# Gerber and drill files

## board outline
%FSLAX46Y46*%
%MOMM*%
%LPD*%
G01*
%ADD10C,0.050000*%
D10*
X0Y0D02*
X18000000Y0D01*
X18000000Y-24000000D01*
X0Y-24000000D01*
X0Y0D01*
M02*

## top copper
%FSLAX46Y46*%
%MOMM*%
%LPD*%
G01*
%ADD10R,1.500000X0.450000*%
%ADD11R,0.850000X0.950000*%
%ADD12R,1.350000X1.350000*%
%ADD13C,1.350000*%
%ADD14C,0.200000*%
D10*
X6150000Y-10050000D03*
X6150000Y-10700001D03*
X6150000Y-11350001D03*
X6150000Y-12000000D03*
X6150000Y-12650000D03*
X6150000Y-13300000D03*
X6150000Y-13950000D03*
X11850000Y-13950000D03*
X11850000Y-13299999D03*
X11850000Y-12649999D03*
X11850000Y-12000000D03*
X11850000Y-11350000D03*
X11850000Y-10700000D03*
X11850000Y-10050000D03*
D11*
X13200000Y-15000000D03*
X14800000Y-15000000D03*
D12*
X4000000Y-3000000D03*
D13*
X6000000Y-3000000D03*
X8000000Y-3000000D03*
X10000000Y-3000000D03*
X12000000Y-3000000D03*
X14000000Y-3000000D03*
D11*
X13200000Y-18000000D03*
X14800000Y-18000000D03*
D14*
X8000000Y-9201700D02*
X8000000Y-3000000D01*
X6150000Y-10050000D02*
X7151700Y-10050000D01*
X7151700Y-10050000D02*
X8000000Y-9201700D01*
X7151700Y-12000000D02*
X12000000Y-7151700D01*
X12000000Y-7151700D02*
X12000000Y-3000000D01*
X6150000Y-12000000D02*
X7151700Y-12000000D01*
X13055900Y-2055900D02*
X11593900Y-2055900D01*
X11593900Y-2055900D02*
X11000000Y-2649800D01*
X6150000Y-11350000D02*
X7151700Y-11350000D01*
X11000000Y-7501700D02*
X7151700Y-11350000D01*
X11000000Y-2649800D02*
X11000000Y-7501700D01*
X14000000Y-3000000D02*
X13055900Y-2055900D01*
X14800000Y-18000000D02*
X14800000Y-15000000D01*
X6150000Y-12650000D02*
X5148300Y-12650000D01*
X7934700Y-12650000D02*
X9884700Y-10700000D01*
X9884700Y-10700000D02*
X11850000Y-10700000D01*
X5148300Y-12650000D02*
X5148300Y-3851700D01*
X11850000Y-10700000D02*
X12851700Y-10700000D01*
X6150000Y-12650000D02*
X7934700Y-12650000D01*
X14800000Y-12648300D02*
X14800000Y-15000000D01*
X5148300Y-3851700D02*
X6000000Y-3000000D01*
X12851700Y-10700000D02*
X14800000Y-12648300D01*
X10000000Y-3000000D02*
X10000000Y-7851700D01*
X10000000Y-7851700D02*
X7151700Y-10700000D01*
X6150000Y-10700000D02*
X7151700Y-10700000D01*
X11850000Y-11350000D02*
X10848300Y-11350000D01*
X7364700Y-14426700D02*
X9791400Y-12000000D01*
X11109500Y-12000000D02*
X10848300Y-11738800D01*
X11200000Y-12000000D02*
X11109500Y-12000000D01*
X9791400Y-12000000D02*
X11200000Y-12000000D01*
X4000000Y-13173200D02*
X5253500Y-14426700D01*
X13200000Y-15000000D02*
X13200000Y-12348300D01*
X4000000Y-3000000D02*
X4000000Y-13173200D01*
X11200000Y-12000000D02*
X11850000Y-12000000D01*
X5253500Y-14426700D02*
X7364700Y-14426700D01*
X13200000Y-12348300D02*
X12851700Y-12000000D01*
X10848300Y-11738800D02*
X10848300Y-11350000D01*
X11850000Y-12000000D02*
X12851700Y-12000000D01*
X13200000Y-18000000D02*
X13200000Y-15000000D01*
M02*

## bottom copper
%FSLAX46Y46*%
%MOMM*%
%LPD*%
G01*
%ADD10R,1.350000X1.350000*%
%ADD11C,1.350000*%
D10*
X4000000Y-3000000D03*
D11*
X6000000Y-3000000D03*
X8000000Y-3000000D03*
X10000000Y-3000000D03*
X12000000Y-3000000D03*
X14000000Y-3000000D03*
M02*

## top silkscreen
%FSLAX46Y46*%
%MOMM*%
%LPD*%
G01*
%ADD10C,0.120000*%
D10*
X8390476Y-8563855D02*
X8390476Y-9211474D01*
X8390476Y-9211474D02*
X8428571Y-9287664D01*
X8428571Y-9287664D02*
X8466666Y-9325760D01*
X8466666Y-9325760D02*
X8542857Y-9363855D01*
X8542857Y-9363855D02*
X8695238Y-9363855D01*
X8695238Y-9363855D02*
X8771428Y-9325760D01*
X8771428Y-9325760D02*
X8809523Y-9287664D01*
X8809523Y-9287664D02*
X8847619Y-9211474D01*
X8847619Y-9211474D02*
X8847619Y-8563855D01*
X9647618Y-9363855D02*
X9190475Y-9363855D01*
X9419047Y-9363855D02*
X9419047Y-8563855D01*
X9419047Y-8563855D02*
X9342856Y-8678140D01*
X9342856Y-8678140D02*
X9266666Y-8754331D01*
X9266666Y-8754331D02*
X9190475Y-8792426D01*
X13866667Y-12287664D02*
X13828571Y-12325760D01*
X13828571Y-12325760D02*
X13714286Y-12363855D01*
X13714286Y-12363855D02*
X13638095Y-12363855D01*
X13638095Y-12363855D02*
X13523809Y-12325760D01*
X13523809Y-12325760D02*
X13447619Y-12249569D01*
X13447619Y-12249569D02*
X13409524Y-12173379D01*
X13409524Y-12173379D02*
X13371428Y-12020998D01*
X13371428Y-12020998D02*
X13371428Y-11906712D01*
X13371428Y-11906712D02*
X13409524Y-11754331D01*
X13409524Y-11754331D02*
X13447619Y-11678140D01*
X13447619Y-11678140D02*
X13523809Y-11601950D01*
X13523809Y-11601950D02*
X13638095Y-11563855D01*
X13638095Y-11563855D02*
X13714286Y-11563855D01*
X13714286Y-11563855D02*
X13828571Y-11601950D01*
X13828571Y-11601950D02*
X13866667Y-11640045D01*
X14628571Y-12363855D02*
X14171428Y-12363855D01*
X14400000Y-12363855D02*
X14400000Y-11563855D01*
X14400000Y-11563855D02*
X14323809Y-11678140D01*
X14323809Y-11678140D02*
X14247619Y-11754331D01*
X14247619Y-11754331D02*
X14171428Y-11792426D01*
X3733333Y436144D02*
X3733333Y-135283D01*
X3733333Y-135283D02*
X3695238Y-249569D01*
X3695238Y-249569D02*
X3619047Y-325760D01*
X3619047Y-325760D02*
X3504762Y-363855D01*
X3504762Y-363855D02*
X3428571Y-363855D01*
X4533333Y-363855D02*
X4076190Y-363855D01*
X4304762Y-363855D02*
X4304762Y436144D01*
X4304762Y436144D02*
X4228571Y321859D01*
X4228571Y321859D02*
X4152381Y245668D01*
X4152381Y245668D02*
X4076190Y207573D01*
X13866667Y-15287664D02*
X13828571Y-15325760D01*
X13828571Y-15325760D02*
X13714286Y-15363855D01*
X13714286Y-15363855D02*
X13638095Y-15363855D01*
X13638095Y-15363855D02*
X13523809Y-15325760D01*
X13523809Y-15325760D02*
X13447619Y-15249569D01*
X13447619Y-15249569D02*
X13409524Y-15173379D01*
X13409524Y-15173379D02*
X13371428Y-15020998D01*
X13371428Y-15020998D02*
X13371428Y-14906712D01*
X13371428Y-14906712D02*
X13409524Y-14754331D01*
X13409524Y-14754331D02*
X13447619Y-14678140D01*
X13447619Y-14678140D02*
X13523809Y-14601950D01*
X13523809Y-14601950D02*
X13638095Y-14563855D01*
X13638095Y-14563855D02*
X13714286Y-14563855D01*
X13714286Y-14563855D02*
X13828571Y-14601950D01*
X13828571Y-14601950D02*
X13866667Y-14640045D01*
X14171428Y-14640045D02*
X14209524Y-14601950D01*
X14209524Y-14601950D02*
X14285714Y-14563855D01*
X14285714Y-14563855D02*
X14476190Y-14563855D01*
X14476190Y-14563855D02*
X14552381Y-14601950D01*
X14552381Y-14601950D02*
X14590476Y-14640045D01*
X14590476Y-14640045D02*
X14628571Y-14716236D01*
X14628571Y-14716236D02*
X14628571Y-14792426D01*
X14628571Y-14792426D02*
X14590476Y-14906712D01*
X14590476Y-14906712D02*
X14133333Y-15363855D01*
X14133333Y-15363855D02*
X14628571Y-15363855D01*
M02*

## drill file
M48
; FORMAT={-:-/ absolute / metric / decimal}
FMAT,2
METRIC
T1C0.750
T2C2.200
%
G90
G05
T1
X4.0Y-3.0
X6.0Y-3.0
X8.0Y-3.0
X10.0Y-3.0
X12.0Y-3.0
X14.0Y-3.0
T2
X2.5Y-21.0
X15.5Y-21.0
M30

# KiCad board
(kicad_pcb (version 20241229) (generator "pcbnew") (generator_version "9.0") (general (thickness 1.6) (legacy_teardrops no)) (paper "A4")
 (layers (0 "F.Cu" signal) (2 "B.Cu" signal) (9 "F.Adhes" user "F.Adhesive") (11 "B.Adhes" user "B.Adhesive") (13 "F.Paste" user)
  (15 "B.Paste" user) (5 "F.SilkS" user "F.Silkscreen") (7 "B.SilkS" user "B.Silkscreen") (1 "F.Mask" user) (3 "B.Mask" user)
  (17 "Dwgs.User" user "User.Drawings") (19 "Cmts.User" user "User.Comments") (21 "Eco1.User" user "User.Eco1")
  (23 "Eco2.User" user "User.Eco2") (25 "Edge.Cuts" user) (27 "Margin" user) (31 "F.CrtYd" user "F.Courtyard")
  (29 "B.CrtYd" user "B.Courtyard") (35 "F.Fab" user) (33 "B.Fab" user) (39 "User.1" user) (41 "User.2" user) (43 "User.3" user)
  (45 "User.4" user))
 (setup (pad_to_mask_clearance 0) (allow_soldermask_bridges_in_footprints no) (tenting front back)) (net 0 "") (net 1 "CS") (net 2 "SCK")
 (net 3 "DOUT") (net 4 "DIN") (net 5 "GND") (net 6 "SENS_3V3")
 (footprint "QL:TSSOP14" (layer "F.Cu") (at 9 12)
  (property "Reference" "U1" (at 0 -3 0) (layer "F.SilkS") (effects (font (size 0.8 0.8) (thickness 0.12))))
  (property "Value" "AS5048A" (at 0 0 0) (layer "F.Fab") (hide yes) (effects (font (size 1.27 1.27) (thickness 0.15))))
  (pad "1" smd rect (at -2.85 -1.95) (size 1.5 0.45) (layers "F.Cu" "F.Mask" "F.Paste") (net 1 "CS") (thermal_bridge_angle 45))
  (pad "2" smd rect (at -2.85 -1.299999) (size 1.5 0.45) (layers "F.Cu" "F.Mask" "F.Paste") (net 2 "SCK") (thermal_bridge_angle 45))
  (pad "3" smd rect (at -2.85 -0.649999) (size 1.5 0.45) (layers "F.Cu" "F.Mask" "F.Paste") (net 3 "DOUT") (thermal_bridge_angle 45))
  (pad "4" smd rect (at -2.85 0) (size 1.5 0.45) (layers "F.Cu" "F.Mask" "F.Paste") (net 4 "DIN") (thermal_bridge_angle 45))
  (pad "5" smd rect (at -2.85 0.65) (size 1.5 0.45) (layers "F.Cu" "F.Mask" "F.Paste") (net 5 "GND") (thermal_bridge_angle 45))
  (pad "6" smd rect (at -2.85 1.3) (size 1.5 0.45) (layers "F.Cu" "F.Mask" "F.Paste") (thermal_bridge_angle 45))
  (pad "7" smd rect (at -2.85 1.95) (size 1.5 0.45) (layers "F.Cu" "F.Mask" "F.Paste") (thermal_bridge_angle 45))
  (pad "8" smd rect (at 2.85 1.95) (size 1.5 0.45) (layers "F.Cu" "F.Mask" "F.Paste") (thermal_bridge_angle 45))
  (pad "9" smd rect (at 2.85 1.299999) (size 1.5 0.45) (layers "F.Cu" "F.Mask" "F.Paste") (thermal_bridge_angle 45))
  (pad "10" smd rect (at 2.85 0.649999) (size 1.5 0.45) (layers "F.Cu" "F.Mask" "F.Paste") (thermal_bridge_angle 45))
  (pad "11" smd rect (at 2.85 0) (size 1.5 0.45) (layers "F.Cu" "F.Mask" "F.Paste") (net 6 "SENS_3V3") (thermal_bridge_angle 45))
  (pad "12" smd rect (at 2.85 -0.65) (size 1.5 0.45) (layers "F.Cu" "F.Mask" "F.Paste") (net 6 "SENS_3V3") (thermal_bridge_angle 45))
  (pad "13" smd rect (at 2.85 -1.3) (size 1.5 0.45) (layers "F.Cu" "F.Mask" "F.Paste") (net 5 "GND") (thermal_bridge_angle 45))
  (pad "14" smd rect (at 2.85 -1.95) (size 1.5 0.45) (layers "F.Cu" "F.Mask" "F.Paste") (thermal_bridge_angle 45)))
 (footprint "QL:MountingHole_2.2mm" (layer "F.Cu") (at 15.5 21)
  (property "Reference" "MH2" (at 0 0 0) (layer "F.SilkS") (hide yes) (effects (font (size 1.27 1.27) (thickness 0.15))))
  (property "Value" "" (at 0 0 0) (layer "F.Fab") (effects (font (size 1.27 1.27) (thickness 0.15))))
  (pad "" np_thru_hole circle (at 0 0) (size 2.2 2.2) (drill 2.2) (layers "*.Cu" "*.Mask")))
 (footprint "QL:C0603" (layer "F.Cu") (at 14 15)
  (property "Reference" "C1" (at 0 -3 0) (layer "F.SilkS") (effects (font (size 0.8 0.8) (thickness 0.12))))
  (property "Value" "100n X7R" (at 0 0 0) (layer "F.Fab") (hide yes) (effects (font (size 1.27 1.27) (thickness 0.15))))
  (pad "1" smd rect (at -0.8 0) (size 0.85 0.95) (layers "F.Cu" "F.Mask" "F.Paste") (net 6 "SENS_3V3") (thermal_bridge_angle 45))
  (pad "2" smd rect (at 0.8 0) (size 0.85 0.95) (layers "F.Cu" "F.Mask" "F.Paste") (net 5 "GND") (thermal_bridge_angle 45)))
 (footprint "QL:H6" (layer "F.Cu") (at 4 3)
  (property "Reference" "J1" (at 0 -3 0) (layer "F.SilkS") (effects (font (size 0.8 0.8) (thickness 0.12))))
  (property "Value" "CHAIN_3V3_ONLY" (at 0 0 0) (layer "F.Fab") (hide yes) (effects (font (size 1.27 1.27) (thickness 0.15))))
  (pad "1" thru_hole rect (at 0 0) (size 1.35 1.35) (drill 0.75) (layers "*.Cu" "*.Mask") (remove_unused_layers no) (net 6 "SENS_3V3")
   (thermal_bridge_angle 45))
  (pad "2" thru_hole circle (at 2 0) (size 1.35 1.35) (drill 0.75) (layers "*.Cu" "*.Mask") (remove_unused_layers no) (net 5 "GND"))
  (pad "3" thru_hole circle (at 4 0) (size 1.35 1.35) (drill 0.75) (layers "*.Cu" "*.Mask") (remove_unused_layers no) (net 1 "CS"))
  (pad "4" thru_hole circle (at 6 0) (size 1.35 1.35) (drill 0.75) (layers "*.Cu" "*.Mask") (remove_unused_layers no) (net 2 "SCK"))
  (pad "5" thru_hole circle (at 8 0) (size 1.35 1.35) (drill 0.75) (layers "*.Cu" "*.Mask") (remove_unused_layers no) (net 4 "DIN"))
  (pad "6" thru_hole circle (at 10 0) (size 1.35 1.35) (drill 0.75) (layers "*.Cu" "*.Mask") (remove_unused_layers no) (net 3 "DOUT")))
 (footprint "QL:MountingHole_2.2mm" (layer "F.Cu") (at 2.5 21)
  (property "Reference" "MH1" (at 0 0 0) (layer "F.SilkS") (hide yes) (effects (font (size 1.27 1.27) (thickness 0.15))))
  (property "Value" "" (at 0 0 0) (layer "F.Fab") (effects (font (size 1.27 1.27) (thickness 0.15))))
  (pad "" np_thru_hole circle (at 0 0) (size 2.2 2.2) (drill 2.2) (layers "*.Cu" "*.Mask")))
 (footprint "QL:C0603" (layer "F.Cu") (at 14 18)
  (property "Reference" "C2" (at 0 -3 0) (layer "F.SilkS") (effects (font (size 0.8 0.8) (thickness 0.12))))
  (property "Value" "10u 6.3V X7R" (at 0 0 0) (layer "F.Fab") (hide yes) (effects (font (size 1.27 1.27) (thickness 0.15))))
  (pad "1" smd rect (at -0.8 0) (size 0.85 0.95) (layers "F.Cu" "F.Mask" "F.Paste") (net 6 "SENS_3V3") (thermal_bridge_angle 45))
  (pad "2" smd rect (at 0.8 0) (size 0.85 0.95) (layers "F.Cu" "F.Mask" "F.Paste") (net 5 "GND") (thermal_bridge_angle 45)))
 (gr_rect (start 0 0) (end 18 24) (stroke (width 0.05) (type default)) (fill no) (layer "Edge.Cuts"))
 (segment (start 8 9.2017) (end 8 3) (width 0.2) (layer "F.Cu") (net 1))
 (segment (start 6.15 10.05) (end 7.1517 10.05) (width 0.2) (layer "F.Cu") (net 1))
 (segment (start 7.1517 10.05) (end 8 9.2017) (width 0.2) (layer "F.Cu") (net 1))
 (segment (start 7.1517 12) (end 12 7.1517) (width 0.2) (layer "F.Cu") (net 4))
 (segment (start 12 7.1517) (end 12 3) (width 0.2) (layer "F.Cu") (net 4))
 (segment (start 6.15 12) (end 7.1517 12) (width 0.2) (layer "F.Cu") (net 4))
 (segment (start 13.0559 2.0559) (end 11.5939 2.0559) (width 0.2) (layer "F.Cu") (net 3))
 (segment (start 11.5939 2.0559) (end 11 2.6498) (width 0.2) (layer "F.Cu") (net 3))
 (segment (start 6.15 11.35) (end 7.1517 11.35) (width 0.2) (layer "F.Cu") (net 3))
 (segment (start 11 7.5017) (end 7.1517 11.35) (width 0.2) (layer "F.Cu") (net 3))
 (segment (start 11 2.6498) (end 11 7.5017) (width 0.2) (layer "F.Cu") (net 3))
 (segment (start 14 3) (end 13.0559 2.0559) (width 0.2) (layer "F.Cu") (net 3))
 (segment (start 14.8 18) (end 14.8 15) (width 0.2) (layer "F.Cu") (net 5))
 (segment (start 6.15 12.65) (end 5.1483 12.65) (width 0.2) (layer "F.Cu") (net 5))
 (segment (start 7.9347 12.65) (end 9.8847 10.7) (width 0.2) (layer "F.Cu") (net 5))
 (segment (start 9.8847 10.7) (end 11.85 10.7) (width 0.2) (layer "F.Cu") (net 5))
 (segment (start 5.1483 12.65) (end 5.1483 3.8517) (width 0.2) (layer "F.Cu") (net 5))
 (segment (start 11.85 10.7) (end 12.8517 10.7) (width 0.2) (layer "F.Cu") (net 5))
 (segment (start 6.15 12.65) (end 7.9347 12.65) (width 0.2) (layer "F.Cu") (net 5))
 (segment (start 14.8 12.6483) (end 14.8 15) (width 0.2) (layer "F.Cu") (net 5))
 (segment (start 5.1483 3.8517) (end 6 3) (width 0.2) (layer "F.Cu") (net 5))
 (segment (start 12.8517 10.7) (end 14.8 12.6483) (width 0.2) (layer "F.Cu") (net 5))
 (segment (start 10 3) (end 10 7.8517) (width 0.2) (layer "F.Cu") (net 2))
 (segment (start 10 7.8517) (end 7.1517 10.7) (width 0.2) (layer "F.Cu") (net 2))
 (segment (start 6.15 10.7) (end 7.1517 10.7) (width 0.2) (layer "F.Cu") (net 2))
 (segment (start 11.85 11.35) (end 10.8483 11.35) (width 0.2) (layer "F.Cu") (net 6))
 (segment (start 7.3647 14.4267) (end 9.7914 12) (width 0.2) (layer "F.Cu") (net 6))
 (segment (start 11.1095 12) (end 10.8483 11.7388) (width 0.2) (layer "F.Cu") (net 6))
 (segment (start 11.2 12) (end 11.1095 12) (width 0.2) (layer "F.Cu") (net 6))
 (segment (start 9.7914 12) (end 11.2 12) (width 0.2) (layer "F.Cu") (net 6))
 (segment (start 4 13.1732) (end 5.2535 14.4267) (width 0.2) (layer "F.Cu") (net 6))
 (segment (start 13.2 15) (end 13.2 12.3483) (width 0.2) (layer "F.Cu") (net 6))
 (segment (start 4 3) (end 4 13.1732) (width 0.2) (layer "F.Cu") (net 6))
 (segment (start 11.2 12) (end 11.85 12) (width 0.2) (layer "F.Cu") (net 6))
 (segment (start 5.2535 14.4267) (end 7.3647 14.4267) (width 0.2) (layer "F.Cu") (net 6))
 (segment (start 13.2 12.3483) (end 12.8517 12) (width 0.2) (layer "F.Cu") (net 6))
 (segment (start 10.8483 11.7388) (end 10.8483 11.35) (width 0.2) (layer "F.Cu") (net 6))
 (segment (start 11.85 12) (end 12.8517 12) (width 0.2) (layer "F.Cu") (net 6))
 (segment (start 13.2 18) (end 13.2 15) (width 0.2) (layer "F.Cu") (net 6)))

